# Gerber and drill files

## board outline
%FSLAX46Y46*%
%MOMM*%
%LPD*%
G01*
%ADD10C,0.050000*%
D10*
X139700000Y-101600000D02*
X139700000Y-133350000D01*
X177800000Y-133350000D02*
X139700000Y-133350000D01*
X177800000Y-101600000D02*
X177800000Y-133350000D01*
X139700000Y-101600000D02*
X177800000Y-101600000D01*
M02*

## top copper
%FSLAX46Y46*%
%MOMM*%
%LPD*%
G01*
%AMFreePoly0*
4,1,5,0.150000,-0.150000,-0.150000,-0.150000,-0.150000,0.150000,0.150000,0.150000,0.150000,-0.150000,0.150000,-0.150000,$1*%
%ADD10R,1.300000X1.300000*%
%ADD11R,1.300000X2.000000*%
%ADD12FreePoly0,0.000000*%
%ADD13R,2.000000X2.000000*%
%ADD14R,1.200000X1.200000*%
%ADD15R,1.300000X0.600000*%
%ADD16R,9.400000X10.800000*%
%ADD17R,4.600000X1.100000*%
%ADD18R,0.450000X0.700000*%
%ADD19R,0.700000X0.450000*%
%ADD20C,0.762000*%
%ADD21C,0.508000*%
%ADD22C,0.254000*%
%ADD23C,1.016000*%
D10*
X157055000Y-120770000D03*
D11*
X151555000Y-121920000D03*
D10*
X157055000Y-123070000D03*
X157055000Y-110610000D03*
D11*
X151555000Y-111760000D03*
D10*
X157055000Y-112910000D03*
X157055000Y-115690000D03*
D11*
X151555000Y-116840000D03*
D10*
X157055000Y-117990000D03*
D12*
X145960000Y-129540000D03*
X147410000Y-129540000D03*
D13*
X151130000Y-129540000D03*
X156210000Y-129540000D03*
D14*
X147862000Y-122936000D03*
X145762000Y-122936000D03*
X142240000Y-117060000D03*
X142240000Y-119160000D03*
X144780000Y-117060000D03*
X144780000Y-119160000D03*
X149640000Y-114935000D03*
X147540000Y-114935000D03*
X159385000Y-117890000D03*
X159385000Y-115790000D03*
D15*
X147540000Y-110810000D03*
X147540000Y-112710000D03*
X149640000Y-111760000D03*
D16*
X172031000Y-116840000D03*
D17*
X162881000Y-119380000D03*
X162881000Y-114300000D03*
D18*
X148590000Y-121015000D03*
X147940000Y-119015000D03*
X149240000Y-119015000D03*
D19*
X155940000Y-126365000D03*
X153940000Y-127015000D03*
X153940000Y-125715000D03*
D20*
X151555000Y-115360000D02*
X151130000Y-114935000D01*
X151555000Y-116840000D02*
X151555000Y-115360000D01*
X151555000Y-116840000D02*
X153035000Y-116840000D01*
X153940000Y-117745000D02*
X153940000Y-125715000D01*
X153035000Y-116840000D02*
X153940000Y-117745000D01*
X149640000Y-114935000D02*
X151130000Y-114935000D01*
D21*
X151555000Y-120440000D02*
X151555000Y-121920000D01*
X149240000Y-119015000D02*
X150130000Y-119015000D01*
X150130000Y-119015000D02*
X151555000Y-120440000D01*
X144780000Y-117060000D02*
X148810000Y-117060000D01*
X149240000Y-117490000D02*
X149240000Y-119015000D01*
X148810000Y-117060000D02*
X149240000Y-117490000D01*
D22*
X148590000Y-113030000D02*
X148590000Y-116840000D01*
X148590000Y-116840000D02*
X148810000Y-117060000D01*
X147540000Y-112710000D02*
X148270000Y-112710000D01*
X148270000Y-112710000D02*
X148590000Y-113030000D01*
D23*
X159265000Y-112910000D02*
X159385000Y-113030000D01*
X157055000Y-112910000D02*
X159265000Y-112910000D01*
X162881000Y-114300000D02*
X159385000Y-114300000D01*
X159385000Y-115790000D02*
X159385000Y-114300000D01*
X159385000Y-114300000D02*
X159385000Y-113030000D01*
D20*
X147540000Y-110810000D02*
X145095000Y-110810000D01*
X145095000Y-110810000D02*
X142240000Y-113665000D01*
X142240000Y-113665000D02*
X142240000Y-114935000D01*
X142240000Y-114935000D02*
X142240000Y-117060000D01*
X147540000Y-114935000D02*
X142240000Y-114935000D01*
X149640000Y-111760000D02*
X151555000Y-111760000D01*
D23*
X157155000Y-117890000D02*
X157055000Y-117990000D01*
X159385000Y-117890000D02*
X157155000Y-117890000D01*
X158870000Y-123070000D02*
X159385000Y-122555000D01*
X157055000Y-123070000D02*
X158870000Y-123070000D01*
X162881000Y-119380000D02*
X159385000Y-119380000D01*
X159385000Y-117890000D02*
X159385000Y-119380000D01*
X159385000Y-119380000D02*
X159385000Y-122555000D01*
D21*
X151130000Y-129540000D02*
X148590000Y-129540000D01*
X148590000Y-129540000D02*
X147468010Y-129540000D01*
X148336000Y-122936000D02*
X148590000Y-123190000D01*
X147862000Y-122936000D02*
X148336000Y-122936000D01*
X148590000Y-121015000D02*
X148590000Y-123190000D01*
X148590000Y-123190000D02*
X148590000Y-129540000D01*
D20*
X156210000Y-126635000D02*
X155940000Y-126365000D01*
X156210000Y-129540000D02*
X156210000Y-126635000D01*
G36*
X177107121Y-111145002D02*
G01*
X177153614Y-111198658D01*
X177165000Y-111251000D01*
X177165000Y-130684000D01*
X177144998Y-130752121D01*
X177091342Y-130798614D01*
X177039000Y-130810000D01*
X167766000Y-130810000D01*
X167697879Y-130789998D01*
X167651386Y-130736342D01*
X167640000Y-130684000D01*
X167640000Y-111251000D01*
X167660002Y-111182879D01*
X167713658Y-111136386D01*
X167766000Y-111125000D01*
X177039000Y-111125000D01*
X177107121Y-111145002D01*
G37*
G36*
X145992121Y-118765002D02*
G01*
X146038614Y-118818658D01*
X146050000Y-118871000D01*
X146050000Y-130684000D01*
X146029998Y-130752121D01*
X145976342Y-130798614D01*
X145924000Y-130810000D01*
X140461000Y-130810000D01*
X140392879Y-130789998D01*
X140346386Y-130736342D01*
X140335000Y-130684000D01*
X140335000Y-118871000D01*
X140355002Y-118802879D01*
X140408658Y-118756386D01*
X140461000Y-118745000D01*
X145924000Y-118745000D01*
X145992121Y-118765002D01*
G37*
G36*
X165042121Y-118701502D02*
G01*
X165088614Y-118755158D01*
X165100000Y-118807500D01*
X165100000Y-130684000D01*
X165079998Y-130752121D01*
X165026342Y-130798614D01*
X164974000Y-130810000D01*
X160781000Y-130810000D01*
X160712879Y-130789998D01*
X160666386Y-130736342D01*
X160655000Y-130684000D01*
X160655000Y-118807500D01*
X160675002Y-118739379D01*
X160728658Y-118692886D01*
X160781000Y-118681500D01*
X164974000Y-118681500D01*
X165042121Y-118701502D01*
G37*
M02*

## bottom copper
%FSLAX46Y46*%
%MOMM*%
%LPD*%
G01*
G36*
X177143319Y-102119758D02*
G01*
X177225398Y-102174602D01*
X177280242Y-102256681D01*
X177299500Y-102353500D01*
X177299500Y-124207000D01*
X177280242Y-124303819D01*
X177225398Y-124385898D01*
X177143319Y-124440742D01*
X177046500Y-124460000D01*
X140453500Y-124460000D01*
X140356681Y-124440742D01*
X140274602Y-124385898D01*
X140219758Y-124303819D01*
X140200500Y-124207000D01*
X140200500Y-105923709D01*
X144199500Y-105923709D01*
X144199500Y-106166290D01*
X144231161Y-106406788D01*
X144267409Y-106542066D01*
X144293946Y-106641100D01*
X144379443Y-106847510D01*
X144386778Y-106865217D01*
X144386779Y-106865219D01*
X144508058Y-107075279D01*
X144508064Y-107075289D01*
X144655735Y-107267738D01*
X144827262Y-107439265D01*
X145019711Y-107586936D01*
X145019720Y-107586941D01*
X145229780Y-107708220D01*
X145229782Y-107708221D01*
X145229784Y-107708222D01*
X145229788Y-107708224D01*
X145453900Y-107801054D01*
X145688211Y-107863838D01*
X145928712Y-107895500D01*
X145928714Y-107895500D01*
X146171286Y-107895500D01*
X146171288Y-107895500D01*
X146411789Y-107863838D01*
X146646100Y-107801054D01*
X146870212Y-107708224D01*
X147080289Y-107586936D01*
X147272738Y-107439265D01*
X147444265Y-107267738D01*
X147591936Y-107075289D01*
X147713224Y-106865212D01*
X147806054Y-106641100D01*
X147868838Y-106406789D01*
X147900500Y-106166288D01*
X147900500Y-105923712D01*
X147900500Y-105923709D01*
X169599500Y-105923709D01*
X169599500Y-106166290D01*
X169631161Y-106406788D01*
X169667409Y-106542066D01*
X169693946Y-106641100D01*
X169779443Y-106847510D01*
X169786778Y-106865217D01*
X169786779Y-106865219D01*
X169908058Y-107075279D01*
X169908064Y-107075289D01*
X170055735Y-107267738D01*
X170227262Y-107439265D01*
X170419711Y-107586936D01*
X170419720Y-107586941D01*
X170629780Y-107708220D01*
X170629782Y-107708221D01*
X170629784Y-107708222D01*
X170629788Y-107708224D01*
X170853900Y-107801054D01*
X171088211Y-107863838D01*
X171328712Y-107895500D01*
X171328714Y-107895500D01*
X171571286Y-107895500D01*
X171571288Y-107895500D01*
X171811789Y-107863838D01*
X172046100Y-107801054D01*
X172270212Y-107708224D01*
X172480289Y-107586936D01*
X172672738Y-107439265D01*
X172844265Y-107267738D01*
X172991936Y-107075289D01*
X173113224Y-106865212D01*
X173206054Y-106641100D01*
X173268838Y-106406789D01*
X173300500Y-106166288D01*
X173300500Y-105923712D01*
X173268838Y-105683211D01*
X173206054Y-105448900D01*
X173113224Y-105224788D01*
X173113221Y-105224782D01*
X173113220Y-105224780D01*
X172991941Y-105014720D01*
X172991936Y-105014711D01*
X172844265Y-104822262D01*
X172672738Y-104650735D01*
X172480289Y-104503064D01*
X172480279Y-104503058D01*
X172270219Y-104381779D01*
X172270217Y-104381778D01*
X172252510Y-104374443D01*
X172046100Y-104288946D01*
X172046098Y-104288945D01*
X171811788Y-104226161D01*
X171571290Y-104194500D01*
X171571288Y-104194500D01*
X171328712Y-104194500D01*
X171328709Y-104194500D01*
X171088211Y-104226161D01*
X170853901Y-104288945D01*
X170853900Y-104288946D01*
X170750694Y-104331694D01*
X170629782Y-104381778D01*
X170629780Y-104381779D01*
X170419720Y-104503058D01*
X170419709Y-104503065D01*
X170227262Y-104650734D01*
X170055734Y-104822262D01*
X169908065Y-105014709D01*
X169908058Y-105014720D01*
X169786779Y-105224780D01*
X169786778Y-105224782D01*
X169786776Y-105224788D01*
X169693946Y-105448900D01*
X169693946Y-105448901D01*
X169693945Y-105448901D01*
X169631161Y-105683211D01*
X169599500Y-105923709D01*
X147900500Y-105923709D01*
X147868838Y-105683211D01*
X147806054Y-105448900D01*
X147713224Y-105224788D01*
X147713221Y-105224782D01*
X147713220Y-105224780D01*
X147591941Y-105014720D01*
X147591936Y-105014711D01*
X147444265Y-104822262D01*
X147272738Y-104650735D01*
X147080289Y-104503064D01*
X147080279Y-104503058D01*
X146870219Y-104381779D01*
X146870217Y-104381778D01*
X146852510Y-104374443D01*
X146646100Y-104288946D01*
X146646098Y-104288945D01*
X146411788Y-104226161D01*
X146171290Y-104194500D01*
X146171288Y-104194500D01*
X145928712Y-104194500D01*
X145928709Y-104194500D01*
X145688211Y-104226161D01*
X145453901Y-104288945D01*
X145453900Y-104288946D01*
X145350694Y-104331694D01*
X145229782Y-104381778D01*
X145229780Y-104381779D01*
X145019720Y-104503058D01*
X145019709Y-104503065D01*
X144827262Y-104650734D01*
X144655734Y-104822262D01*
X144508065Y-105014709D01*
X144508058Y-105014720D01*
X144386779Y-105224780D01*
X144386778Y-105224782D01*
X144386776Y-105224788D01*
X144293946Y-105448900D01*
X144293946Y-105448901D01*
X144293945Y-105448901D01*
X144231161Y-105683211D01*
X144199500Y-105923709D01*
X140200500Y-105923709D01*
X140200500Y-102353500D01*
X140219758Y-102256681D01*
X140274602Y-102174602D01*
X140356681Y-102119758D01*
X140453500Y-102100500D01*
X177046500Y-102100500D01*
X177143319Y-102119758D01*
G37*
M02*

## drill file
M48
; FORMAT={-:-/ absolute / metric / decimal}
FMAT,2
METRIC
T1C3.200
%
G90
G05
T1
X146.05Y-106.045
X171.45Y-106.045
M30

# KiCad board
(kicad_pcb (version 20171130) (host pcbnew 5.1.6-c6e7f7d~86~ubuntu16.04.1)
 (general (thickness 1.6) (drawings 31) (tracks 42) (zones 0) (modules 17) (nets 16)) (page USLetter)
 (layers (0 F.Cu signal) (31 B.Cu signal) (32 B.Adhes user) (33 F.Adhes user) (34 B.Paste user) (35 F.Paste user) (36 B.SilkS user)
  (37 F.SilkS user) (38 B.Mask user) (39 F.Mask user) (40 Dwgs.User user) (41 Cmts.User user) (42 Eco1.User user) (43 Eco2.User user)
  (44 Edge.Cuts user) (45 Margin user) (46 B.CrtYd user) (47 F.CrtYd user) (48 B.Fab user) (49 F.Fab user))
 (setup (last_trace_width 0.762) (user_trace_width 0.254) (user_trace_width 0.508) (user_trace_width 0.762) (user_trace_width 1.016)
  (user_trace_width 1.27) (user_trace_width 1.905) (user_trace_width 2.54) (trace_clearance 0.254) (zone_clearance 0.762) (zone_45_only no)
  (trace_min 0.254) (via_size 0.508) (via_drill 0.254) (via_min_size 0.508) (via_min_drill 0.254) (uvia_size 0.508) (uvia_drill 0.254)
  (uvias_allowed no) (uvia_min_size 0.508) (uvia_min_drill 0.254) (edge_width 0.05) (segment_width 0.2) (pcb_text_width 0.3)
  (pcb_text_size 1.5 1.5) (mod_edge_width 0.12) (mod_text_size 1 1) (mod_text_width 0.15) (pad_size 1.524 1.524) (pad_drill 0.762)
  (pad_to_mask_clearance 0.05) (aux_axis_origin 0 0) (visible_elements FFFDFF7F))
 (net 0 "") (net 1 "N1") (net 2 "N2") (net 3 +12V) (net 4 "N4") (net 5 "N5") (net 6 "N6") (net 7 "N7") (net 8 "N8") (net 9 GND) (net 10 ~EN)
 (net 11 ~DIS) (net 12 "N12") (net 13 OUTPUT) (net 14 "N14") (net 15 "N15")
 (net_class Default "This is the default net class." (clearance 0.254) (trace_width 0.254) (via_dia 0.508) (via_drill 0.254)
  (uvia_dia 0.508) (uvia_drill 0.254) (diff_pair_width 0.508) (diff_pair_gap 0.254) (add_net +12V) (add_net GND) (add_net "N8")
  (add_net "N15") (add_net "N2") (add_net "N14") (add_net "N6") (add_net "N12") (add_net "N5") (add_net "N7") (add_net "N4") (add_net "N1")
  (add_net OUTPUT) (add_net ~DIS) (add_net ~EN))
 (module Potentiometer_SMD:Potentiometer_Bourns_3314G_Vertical (layer F.Cu) (at 154.305 121.92 270)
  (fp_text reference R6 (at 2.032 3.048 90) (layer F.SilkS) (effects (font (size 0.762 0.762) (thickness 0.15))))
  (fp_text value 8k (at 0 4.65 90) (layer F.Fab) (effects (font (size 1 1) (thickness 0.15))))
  (pad 3 smd rect (at -1.15 -2.75 270) (size 1.3 1.3) (layers F.Cu F.Paste F.Mask) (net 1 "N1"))
  (pad 2 smd rect (at 0 2.75 270) (size 2 1.3) (layers F.Cu F.Paste F.Mask) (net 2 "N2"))
  (pad 1 smd rect (at 1.15 -2.75 270) (size 1.3 1.3) (layers F.Cu F.Paste F.Mask) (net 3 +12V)))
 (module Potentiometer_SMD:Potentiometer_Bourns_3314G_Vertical (layer F.Cu) (at 154.305 111.76 270)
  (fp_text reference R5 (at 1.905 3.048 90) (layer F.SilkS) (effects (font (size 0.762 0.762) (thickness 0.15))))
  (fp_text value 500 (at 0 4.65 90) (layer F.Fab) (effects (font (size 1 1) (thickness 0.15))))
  (pad 3 smd rect (at -1.15 -2.75 270) (size 1.3 1.3) (layers F.Cu F.Paste F.Mask) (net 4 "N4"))
  (pad 2 smd rect (at 0 2.75 270) (size 2 1.3) (layers F.Cu F.Paste F.Mask) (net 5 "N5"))
  (pad 1 smd rect (at 1.15 -2.75 270) (size 1.3 1.3) (layers F.Cu F.Paste F.Mask) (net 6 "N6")))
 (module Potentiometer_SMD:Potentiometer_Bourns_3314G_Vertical (layer F.Cu) (at 154.305 116.84 270)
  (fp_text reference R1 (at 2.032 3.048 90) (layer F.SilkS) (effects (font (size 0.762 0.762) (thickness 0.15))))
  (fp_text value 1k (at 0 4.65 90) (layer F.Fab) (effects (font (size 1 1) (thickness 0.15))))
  (pad 3 smd rect (at -1.15 -2.75 270) (size 1.3 1.3) (layers F.Cu F.Paste F.Mask) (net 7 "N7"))
  (pad 2 smd rect (at 0 2.75 270) (size 2 1.3) (layers F.Cu F.Paste F.Mask) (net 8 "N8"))
  (pad 1 smd rect (at 1.15 -2.75 270) (size 1.3 1.3) (layers F.Cu F.Paste F.Mask) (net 3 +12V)))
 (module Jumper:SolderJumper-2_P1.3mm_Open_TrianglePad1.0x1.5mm (layer F.Cu) (at 146.685 129.54)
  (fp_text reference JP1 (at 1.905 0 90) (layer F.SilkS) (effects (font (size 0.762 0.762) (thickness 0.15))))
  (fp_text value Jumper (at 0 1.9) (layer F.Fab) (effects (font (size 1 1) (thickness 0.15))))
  (pad 1 smd custom (at -0.725 0) (size 0.3 0.3) (layers F.Cu F.Mask) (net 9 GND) (zone_connect 2)
   (options (clearance outline) (anchor rect)) (primitives))
  (pad 2 smd custom (at 0.725 0) (size 0.3 0.3) (layers F.Cu F.Mask) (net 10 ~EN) (zone_connect 2)
   (options (clearance outline) (anchor rect)) (primitives)))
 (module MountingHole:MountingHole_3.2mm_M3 (layer F.Cu) (at 171.45 106.045)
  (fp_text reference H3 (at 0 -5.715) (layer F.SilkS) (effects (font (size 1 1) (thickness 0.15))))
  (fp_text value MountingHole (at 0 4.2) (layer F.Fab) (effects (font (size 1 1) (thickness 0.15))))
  (pad 1 np_thru_hole circle (at 0 0) (size 3.2 3.2) (drill 3.2) (layers *.Cu *.Mask)))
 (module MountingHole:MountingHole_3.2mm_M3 (layer F.Cu) (at 146.05 106.045)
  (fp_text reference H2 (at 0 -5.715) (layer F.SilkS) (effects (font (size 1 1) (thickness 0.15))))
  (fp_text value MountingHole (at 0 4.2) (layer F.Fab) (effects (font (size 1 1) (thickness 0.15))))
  (pad 1 np_thru_hole circle (at 0 0) (size 3.2 3.2) (drill 3.2) (layers *.Cu *.Mask)))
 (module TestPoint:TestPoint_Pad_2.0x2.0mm (layer F.Cu) (at 151.13 129.54 180)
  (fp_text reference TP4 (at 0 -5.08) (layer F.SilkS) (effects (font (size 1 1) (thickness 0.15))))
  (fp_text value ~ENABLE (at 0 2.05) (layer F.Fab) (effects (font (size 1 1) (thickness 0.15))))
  (pad 1 smd rect (at 0 0 180) (size 2 2) (layers F.Cu F.Mask) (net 10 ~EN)))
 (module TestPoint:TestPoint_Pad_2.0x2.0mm (layer F.Cu) (at 156.21 129.54 180)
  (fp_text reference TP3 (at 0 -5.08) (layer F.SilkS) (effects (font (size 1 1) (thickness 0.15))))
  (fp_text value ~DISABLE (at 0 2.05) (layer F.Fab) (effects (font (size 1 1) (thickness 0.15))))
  (pad 1 smd rect (at 0 0 180) (size 2 2) (layers F.Cu F.Mask) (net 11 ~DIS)))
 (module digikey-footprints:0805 (layer F.Cu) (at 146.812 122.936 180)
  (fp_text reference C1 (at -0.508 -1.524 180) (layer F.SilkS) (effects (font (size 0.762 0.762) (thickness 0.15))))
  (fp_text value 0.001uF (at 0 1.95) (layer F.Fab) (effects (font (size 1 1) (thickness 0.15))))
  (pad 1 smd rect (at -1.05 0 180) (size 1.2 1.2) (layers F.Cu F.Paste F.Mask) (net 10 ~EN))
  (pad 2 smd rect (at 1.05 0 180) (size 1.2 1.2) (layers F.Cu F.Paste F.Mask) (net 9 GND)))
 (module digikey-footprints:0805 (layer F.Cu) (at 142.24 118.11 270)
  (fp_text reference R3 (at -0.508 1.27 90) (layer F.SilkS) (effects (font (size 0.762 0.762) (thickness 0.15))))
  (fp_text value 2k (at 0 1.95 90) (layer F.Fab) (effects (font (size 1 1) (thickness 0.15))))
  (pad 1 smd rect (at -1.05 0 270) (size 1.2 1.2) (layers F.Cu F.Paste F.Mask) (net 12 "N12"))
  (pad 2 smd rect (at 1.05 0 270) (size 1.2 1.2) (layers F.Cu F.Paste F.Mask) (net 9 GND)))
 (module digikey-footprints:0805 (layer F.Cu) (at 144.78 118.11 270)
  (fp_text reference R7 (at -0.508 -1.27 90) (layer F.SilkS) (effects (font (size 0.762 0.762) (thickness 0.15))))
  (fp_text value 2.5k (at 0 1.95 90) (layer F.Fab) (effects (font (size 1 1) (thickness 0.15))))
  (pad 1 smd rect (at -1.05 0 270) (size 1.2 1.2) (layers F.Cu F.Paste F.Mask) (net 2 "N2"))
  (pad 2 smd rect (at 1.05 0 270) (size 1.2 1.2) (layers F.Cu F.Paste F.Mask) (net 9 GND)))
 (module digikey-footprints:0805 (layer F.Cu) (at 148.59 114.935 180)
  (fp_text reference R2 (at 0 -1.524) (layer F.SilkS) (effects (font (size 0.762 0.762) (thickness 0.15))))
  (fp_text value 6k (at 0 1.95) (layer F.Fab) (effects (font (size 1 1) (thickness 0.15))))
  (pad 1 smd rect (at -1.05 0 180) (size 1.2 1.2) (layers F.Cu F.Paste F.Mask) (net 8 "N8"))
  (pad 2 smd rect (at 1.05 0 180) (size 1.2 1.2) (layers F.Cu F.Paste F.Mask) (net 12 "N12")))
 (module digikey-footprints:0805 (layer F.Cu) (at 159.385 116.84 90)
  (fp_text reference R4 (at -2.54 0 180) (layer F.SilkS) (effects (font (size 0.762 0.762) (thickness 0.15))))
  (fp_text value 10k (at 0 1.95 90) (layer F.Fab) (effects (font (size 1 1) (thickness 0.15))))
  (pad 1 smd rect (at -1.05 0 90) (size 1.2 1.2) (layers F.Cu F.Paste F.Mask) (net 3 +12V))
  (pad 2 smd rect (at 1.05 0 90) (size 1.2 1.2) (layers F.Cu F.Paste F.Mask) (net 6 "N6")))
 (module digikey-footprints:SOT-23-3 (layer F.Cu) (at 148.59 111.76)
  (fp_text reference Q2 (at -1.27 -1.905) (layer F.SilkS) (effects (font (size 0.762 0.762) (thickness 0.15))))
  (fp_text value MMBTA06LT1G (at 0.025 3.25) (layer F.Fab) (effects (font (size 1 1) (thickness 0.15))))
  (pad 1 smd rect (at -1.05 -0.95) (size 1.3 0.6) (layers F.Cu F.Paste F.Mask) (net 12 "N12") (solder_mask_margin 0.07))
  (pad 2 smd rect (at -1.05 0.95) (size 1.3 0.6) (layers F.Cu F.Paste F.Mask) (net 2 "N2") (solder_mask_margin 0.07))
  (pad 3 smd rect (at 1.05 0) (size 1.3 0.6) (layers F.Cu F.Paste F.Mask) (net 5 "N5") (solder_mask_margin 0.07)))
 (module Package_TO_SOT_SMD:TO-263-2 (layer F.Cu) (at 168.656 116.84)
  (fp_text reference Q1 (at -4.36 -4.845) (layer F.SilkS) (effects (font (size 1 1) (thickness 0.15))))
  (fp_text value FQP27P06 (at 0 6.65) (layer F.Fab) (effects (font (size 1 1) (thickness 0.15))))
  (pad "" smd rect (at 0.95 2.775) (size 4.55 5.25) (layers F.Paste))
  (pad "" smd rect (at 5.8 -2.775) (size 4.55 5.25) (layers F.Paste))
  (pad "" smd rect (at 0.95 -2.775) (size 4.55 5.25) (layers F.Paste))
  (pad "" smd rect (at 5.8 2.775) (size 4.55 5.25) (layers F.Paste))
  (pad 2 smd rect (at 3.375 0) (size 9.4 10.8) (layers F.Cu F.Mask) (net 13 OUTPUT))
  (pad 3 smd rect (at -5.775 2.54) (size 4.6 1.1) (layers F.Cu F.Paste F.Mask) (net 3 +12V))
  (pad 1 smd rect (at -5.775 -2.54) (size 4.6 1.1) (layers F.Cu F.Paste F.Mask) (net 6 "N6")))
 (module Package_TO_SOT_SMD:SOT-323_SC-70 (layer F.Cu) (at 148.59 120.015 270)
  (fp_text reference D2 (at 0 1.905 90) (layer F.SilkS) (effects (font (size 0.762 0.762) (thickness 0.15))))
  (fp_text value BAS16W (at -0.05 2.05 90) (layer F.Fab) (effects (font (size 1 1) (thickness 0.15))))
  (pad 3 smd rect (at 1 0 180) (size 0.45 0.7) (layers F.Cu F.Paste F.Mask) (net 10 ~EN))
  (pad 2 smd rect (at -1 0.65 180) (size 0.45 0.7) (layers F.Cu F.Paste F.Mask) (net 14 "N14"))
  (pad 1 smd rect (at -1 -0.65 180) (size 0.45 0.7) (layers F.Cu F.Paste F.Mask) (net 2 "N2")))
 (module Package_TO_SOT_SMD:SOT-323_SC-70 (layer F.Cu) (at 154.94 126.365)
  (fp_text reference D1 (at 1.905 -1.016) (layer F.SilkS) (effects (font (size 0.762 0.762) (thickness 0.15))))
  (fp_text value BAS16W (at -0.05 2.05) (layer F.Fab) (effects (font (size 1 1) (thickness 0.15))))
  (pad 3 smd rect (at 1 0 270) (size 0.45 0.7) (layers F.Cu F.Paste F.Mask) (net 11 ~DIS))
  (pad 2 smd rect (at -1 0.65 270) (size 0.45 0.7) (layers F.Cu F.Paste F.Mask) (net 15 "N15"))
  (pad 1 smd rect (at -1 -0.65 270) (size 0.45 0.7) (layers F.Cu F.Paste F.Mask) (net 8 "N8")))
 (gr_line (start 139.7 101.6) (end 139.7 133.35) (layer Edge.Cuts) (width 0.05))
 (gr_line (start 177.8 133.35) (end 139.7 133.35) (layer Edge.Cuts) (width 0.05))
 (gr_line (start 177.8 101.6) (end 177.8 133.35) (layer Edge.Cuts) (width 0.05))
 (gr_line (start 139.7 101.6) (end 177.8 101.6) (layer Edge.Cuts) (width 0.05))
 (segment (start 151.555 115.36) (end 151.13 114.935) (width 0.762) (layer F.Cu) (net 8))
 (segment (start 151.555 116.84) (end 151.555 115.36) (width 0.762) (layer F.Cu) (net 8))
 (segment (start 151.555 116.84) (end 153.035 116.84) (width 0.762) (layer F.Cu) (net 8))
 (segment (start 153.94 117.745) (end 153.94 125.715) (width 0.762) (layer F.Cu) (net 8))
 (segment (start 153.035 116.84) (end 153.94 117.745) (width 0.762) (layer F.Cu) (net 8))
 (segment (start 149.64 114.935) (end 151.13 114.935) (width 0.762) (layer F.Cu) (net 8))
 (segment (start 151.555 120.44) (end 151.555 121.92) (width 0.508) (layer F.Cu) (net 2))
 (segment (start 149.24 119.015) (end 150.13 119.015) (width 0.508) (layer F.Cu) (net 2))
 (segment (start 150.13 119.015) (end 151.555 120.44) (width 0.508) (layer F.Cu) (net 2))
 (segment (start 144.78 117.06) (end 148.81 117.06) (width 0.508) (layer F.Cu) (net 2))
 (segment (start 149.24 117.49) (end 149.24 119.015) (width 0.508) (layer F.Cu) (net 2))
 (segment (start 148.81 117.06) (end 149.24 117.49) (width 0.508) (layer F.Cu) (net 2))
 (segment (start 148.59 113.03) (end 148.59 116.84) (width 0.254) (layer F.Cu) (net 2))
 (segment (start 148.59 116.84) (end 148.81 117.06) (width 0.254) (layer F.Cu) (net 2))
 (segment (start 147.54 112.71) (end 148.27 112.71) (width 0.254) (layer F.Cu) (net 2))
 (segment (start 148.27 112.71) (end 148.59 113.03) (width 0.254) (layer F.Cu) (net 2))
 (segment (start 159.265 112.91) (end 159.385 113.03) (width 1.016) (layer F.Cu) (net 6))
 (segment (start 157.055 112.91) (end 159.265 112.91) (width 1.016) (layer F.Cu) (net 6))
 (segment (start 162.881 114.3) (end 159.385 114.3) (width 1.016) (layer F.Cu) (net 6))
 (segment (start 159.385 115.79) (end 159.385 114.3) (width 1.016) (layer F.Cu) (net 6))
 (segment (start 159.385 114.3) (end 159.385 113.03) (width 1.016) (layer F.Cu) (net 6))
 (segment (start 147.54 110.81) (end 145.095 110.81) (width 0.762) (layer F.Cu) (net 12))
 (segment (start 145.095 110.81) (end 142.24 113.665) (width 0.762) (layer F.Cu) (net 12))
 (segment (start 142.24 113.665) (end 142.24 114.935) (width 0.762) (layer F.Cu) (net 12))
 (segment (start 142.24 114.935) (end 142.24 117.06) (width 0.762) (layer F.Cu) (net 12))
 (segment (start 147.54 114.935) (end 142.24 114.935) (width 0.762) (layer F.Cu) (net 12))
 (segment (start 149.64 111.76) (end 151.555 111.76) (width 0.762) (layer F.Cu) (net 5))
 (segment (start 157.155 117.89) (end 157.055 117.99) (width 1.016) (layer F.Cu) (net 3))
 (segment (start 159.385 117.89) (end 157.155 117.89) (width 1.016) (layer F.Cu) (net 3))
 (segment (start 158.87 123.07) (end 159.385 122.555) (width 1.016) (layer F.Cu) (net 3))
 (segment (start 157.055 123.07) (end 158.87 123.07) (width 1.016) (layer F.Cu) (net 3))
 (segment (start 162.881 119.38) (end 159.385 119.38) (width 1.016) (layer F.Cu) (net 3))
 (segment (start 159.385 117.89) (end 159.385 119.38) (width 1.016) (layer F.Cu) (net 3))
 (segment (start 159.385 119.38) (end 159.385 122.555) (width 1.016) (layer F.Cu) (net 3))
 (segment (start 151.13 129.54) (end 148.59 129.54) (width 0.508) (layer F.Cu) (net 10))
 (segment (start 148.59 129.54) (end 147.46801 129.54) (width 0.508) (layer F.Cu) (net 10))
 (segment (start 148.336 122.936) (end 148.59 123.19) (width 0.508) (layer F.Cu) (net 10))
 (segment (start 147.862 122.936) (end 148.336 122.936) (width 0.508) (layer F.Cu) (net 10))
 (segment (start 148.59 121.015) (end 148.59 123.19) (width 0.508) (layer F.Cu) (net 10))
 (segment (start 148.59 123.19) (end 148.59 129.54) (width 0.508) (layer F.Cu) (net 10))
 (segment (start 156.21 126.635) (end 155.94 126.365) (width 0.762) (layer F.Cu) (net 11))
 (segment (start 156.21 129.54) (end 156.21 126.635) (width 0.762) (layer F.Cu) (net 11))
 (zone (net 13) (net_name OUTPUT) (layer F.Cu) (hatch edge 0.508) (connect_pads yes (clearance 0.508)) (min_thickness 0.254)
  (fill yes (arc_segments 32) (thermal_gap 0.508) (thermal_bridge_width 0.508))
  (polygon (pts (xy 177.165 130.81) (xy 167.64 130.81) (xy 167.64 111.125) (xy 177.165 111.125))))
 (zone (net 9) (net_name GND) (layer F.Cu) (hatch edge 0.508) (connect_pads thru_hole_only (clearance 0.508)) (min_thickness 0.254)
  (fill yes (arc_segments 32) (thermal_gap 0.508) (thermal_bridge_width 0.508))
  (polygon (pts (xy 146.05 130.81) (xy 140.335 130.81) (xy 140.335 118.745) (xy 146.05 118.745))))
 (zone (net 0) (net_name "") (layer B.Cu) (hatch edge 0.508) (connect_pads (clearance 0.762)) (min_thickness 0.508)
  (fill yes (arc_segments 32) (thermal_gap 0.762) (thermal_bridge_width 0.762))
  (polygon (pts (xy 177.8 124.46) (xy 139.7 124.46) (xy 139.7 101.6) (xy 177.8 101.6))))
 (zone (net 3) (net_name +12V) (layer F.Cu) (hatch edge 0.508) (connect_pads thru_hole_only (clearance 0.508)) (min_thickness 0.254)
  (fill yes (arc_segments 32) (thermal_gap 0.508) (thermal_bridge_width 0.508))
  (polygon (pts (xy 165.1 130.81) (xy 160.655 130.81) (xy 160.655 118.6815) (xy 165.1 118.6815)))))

